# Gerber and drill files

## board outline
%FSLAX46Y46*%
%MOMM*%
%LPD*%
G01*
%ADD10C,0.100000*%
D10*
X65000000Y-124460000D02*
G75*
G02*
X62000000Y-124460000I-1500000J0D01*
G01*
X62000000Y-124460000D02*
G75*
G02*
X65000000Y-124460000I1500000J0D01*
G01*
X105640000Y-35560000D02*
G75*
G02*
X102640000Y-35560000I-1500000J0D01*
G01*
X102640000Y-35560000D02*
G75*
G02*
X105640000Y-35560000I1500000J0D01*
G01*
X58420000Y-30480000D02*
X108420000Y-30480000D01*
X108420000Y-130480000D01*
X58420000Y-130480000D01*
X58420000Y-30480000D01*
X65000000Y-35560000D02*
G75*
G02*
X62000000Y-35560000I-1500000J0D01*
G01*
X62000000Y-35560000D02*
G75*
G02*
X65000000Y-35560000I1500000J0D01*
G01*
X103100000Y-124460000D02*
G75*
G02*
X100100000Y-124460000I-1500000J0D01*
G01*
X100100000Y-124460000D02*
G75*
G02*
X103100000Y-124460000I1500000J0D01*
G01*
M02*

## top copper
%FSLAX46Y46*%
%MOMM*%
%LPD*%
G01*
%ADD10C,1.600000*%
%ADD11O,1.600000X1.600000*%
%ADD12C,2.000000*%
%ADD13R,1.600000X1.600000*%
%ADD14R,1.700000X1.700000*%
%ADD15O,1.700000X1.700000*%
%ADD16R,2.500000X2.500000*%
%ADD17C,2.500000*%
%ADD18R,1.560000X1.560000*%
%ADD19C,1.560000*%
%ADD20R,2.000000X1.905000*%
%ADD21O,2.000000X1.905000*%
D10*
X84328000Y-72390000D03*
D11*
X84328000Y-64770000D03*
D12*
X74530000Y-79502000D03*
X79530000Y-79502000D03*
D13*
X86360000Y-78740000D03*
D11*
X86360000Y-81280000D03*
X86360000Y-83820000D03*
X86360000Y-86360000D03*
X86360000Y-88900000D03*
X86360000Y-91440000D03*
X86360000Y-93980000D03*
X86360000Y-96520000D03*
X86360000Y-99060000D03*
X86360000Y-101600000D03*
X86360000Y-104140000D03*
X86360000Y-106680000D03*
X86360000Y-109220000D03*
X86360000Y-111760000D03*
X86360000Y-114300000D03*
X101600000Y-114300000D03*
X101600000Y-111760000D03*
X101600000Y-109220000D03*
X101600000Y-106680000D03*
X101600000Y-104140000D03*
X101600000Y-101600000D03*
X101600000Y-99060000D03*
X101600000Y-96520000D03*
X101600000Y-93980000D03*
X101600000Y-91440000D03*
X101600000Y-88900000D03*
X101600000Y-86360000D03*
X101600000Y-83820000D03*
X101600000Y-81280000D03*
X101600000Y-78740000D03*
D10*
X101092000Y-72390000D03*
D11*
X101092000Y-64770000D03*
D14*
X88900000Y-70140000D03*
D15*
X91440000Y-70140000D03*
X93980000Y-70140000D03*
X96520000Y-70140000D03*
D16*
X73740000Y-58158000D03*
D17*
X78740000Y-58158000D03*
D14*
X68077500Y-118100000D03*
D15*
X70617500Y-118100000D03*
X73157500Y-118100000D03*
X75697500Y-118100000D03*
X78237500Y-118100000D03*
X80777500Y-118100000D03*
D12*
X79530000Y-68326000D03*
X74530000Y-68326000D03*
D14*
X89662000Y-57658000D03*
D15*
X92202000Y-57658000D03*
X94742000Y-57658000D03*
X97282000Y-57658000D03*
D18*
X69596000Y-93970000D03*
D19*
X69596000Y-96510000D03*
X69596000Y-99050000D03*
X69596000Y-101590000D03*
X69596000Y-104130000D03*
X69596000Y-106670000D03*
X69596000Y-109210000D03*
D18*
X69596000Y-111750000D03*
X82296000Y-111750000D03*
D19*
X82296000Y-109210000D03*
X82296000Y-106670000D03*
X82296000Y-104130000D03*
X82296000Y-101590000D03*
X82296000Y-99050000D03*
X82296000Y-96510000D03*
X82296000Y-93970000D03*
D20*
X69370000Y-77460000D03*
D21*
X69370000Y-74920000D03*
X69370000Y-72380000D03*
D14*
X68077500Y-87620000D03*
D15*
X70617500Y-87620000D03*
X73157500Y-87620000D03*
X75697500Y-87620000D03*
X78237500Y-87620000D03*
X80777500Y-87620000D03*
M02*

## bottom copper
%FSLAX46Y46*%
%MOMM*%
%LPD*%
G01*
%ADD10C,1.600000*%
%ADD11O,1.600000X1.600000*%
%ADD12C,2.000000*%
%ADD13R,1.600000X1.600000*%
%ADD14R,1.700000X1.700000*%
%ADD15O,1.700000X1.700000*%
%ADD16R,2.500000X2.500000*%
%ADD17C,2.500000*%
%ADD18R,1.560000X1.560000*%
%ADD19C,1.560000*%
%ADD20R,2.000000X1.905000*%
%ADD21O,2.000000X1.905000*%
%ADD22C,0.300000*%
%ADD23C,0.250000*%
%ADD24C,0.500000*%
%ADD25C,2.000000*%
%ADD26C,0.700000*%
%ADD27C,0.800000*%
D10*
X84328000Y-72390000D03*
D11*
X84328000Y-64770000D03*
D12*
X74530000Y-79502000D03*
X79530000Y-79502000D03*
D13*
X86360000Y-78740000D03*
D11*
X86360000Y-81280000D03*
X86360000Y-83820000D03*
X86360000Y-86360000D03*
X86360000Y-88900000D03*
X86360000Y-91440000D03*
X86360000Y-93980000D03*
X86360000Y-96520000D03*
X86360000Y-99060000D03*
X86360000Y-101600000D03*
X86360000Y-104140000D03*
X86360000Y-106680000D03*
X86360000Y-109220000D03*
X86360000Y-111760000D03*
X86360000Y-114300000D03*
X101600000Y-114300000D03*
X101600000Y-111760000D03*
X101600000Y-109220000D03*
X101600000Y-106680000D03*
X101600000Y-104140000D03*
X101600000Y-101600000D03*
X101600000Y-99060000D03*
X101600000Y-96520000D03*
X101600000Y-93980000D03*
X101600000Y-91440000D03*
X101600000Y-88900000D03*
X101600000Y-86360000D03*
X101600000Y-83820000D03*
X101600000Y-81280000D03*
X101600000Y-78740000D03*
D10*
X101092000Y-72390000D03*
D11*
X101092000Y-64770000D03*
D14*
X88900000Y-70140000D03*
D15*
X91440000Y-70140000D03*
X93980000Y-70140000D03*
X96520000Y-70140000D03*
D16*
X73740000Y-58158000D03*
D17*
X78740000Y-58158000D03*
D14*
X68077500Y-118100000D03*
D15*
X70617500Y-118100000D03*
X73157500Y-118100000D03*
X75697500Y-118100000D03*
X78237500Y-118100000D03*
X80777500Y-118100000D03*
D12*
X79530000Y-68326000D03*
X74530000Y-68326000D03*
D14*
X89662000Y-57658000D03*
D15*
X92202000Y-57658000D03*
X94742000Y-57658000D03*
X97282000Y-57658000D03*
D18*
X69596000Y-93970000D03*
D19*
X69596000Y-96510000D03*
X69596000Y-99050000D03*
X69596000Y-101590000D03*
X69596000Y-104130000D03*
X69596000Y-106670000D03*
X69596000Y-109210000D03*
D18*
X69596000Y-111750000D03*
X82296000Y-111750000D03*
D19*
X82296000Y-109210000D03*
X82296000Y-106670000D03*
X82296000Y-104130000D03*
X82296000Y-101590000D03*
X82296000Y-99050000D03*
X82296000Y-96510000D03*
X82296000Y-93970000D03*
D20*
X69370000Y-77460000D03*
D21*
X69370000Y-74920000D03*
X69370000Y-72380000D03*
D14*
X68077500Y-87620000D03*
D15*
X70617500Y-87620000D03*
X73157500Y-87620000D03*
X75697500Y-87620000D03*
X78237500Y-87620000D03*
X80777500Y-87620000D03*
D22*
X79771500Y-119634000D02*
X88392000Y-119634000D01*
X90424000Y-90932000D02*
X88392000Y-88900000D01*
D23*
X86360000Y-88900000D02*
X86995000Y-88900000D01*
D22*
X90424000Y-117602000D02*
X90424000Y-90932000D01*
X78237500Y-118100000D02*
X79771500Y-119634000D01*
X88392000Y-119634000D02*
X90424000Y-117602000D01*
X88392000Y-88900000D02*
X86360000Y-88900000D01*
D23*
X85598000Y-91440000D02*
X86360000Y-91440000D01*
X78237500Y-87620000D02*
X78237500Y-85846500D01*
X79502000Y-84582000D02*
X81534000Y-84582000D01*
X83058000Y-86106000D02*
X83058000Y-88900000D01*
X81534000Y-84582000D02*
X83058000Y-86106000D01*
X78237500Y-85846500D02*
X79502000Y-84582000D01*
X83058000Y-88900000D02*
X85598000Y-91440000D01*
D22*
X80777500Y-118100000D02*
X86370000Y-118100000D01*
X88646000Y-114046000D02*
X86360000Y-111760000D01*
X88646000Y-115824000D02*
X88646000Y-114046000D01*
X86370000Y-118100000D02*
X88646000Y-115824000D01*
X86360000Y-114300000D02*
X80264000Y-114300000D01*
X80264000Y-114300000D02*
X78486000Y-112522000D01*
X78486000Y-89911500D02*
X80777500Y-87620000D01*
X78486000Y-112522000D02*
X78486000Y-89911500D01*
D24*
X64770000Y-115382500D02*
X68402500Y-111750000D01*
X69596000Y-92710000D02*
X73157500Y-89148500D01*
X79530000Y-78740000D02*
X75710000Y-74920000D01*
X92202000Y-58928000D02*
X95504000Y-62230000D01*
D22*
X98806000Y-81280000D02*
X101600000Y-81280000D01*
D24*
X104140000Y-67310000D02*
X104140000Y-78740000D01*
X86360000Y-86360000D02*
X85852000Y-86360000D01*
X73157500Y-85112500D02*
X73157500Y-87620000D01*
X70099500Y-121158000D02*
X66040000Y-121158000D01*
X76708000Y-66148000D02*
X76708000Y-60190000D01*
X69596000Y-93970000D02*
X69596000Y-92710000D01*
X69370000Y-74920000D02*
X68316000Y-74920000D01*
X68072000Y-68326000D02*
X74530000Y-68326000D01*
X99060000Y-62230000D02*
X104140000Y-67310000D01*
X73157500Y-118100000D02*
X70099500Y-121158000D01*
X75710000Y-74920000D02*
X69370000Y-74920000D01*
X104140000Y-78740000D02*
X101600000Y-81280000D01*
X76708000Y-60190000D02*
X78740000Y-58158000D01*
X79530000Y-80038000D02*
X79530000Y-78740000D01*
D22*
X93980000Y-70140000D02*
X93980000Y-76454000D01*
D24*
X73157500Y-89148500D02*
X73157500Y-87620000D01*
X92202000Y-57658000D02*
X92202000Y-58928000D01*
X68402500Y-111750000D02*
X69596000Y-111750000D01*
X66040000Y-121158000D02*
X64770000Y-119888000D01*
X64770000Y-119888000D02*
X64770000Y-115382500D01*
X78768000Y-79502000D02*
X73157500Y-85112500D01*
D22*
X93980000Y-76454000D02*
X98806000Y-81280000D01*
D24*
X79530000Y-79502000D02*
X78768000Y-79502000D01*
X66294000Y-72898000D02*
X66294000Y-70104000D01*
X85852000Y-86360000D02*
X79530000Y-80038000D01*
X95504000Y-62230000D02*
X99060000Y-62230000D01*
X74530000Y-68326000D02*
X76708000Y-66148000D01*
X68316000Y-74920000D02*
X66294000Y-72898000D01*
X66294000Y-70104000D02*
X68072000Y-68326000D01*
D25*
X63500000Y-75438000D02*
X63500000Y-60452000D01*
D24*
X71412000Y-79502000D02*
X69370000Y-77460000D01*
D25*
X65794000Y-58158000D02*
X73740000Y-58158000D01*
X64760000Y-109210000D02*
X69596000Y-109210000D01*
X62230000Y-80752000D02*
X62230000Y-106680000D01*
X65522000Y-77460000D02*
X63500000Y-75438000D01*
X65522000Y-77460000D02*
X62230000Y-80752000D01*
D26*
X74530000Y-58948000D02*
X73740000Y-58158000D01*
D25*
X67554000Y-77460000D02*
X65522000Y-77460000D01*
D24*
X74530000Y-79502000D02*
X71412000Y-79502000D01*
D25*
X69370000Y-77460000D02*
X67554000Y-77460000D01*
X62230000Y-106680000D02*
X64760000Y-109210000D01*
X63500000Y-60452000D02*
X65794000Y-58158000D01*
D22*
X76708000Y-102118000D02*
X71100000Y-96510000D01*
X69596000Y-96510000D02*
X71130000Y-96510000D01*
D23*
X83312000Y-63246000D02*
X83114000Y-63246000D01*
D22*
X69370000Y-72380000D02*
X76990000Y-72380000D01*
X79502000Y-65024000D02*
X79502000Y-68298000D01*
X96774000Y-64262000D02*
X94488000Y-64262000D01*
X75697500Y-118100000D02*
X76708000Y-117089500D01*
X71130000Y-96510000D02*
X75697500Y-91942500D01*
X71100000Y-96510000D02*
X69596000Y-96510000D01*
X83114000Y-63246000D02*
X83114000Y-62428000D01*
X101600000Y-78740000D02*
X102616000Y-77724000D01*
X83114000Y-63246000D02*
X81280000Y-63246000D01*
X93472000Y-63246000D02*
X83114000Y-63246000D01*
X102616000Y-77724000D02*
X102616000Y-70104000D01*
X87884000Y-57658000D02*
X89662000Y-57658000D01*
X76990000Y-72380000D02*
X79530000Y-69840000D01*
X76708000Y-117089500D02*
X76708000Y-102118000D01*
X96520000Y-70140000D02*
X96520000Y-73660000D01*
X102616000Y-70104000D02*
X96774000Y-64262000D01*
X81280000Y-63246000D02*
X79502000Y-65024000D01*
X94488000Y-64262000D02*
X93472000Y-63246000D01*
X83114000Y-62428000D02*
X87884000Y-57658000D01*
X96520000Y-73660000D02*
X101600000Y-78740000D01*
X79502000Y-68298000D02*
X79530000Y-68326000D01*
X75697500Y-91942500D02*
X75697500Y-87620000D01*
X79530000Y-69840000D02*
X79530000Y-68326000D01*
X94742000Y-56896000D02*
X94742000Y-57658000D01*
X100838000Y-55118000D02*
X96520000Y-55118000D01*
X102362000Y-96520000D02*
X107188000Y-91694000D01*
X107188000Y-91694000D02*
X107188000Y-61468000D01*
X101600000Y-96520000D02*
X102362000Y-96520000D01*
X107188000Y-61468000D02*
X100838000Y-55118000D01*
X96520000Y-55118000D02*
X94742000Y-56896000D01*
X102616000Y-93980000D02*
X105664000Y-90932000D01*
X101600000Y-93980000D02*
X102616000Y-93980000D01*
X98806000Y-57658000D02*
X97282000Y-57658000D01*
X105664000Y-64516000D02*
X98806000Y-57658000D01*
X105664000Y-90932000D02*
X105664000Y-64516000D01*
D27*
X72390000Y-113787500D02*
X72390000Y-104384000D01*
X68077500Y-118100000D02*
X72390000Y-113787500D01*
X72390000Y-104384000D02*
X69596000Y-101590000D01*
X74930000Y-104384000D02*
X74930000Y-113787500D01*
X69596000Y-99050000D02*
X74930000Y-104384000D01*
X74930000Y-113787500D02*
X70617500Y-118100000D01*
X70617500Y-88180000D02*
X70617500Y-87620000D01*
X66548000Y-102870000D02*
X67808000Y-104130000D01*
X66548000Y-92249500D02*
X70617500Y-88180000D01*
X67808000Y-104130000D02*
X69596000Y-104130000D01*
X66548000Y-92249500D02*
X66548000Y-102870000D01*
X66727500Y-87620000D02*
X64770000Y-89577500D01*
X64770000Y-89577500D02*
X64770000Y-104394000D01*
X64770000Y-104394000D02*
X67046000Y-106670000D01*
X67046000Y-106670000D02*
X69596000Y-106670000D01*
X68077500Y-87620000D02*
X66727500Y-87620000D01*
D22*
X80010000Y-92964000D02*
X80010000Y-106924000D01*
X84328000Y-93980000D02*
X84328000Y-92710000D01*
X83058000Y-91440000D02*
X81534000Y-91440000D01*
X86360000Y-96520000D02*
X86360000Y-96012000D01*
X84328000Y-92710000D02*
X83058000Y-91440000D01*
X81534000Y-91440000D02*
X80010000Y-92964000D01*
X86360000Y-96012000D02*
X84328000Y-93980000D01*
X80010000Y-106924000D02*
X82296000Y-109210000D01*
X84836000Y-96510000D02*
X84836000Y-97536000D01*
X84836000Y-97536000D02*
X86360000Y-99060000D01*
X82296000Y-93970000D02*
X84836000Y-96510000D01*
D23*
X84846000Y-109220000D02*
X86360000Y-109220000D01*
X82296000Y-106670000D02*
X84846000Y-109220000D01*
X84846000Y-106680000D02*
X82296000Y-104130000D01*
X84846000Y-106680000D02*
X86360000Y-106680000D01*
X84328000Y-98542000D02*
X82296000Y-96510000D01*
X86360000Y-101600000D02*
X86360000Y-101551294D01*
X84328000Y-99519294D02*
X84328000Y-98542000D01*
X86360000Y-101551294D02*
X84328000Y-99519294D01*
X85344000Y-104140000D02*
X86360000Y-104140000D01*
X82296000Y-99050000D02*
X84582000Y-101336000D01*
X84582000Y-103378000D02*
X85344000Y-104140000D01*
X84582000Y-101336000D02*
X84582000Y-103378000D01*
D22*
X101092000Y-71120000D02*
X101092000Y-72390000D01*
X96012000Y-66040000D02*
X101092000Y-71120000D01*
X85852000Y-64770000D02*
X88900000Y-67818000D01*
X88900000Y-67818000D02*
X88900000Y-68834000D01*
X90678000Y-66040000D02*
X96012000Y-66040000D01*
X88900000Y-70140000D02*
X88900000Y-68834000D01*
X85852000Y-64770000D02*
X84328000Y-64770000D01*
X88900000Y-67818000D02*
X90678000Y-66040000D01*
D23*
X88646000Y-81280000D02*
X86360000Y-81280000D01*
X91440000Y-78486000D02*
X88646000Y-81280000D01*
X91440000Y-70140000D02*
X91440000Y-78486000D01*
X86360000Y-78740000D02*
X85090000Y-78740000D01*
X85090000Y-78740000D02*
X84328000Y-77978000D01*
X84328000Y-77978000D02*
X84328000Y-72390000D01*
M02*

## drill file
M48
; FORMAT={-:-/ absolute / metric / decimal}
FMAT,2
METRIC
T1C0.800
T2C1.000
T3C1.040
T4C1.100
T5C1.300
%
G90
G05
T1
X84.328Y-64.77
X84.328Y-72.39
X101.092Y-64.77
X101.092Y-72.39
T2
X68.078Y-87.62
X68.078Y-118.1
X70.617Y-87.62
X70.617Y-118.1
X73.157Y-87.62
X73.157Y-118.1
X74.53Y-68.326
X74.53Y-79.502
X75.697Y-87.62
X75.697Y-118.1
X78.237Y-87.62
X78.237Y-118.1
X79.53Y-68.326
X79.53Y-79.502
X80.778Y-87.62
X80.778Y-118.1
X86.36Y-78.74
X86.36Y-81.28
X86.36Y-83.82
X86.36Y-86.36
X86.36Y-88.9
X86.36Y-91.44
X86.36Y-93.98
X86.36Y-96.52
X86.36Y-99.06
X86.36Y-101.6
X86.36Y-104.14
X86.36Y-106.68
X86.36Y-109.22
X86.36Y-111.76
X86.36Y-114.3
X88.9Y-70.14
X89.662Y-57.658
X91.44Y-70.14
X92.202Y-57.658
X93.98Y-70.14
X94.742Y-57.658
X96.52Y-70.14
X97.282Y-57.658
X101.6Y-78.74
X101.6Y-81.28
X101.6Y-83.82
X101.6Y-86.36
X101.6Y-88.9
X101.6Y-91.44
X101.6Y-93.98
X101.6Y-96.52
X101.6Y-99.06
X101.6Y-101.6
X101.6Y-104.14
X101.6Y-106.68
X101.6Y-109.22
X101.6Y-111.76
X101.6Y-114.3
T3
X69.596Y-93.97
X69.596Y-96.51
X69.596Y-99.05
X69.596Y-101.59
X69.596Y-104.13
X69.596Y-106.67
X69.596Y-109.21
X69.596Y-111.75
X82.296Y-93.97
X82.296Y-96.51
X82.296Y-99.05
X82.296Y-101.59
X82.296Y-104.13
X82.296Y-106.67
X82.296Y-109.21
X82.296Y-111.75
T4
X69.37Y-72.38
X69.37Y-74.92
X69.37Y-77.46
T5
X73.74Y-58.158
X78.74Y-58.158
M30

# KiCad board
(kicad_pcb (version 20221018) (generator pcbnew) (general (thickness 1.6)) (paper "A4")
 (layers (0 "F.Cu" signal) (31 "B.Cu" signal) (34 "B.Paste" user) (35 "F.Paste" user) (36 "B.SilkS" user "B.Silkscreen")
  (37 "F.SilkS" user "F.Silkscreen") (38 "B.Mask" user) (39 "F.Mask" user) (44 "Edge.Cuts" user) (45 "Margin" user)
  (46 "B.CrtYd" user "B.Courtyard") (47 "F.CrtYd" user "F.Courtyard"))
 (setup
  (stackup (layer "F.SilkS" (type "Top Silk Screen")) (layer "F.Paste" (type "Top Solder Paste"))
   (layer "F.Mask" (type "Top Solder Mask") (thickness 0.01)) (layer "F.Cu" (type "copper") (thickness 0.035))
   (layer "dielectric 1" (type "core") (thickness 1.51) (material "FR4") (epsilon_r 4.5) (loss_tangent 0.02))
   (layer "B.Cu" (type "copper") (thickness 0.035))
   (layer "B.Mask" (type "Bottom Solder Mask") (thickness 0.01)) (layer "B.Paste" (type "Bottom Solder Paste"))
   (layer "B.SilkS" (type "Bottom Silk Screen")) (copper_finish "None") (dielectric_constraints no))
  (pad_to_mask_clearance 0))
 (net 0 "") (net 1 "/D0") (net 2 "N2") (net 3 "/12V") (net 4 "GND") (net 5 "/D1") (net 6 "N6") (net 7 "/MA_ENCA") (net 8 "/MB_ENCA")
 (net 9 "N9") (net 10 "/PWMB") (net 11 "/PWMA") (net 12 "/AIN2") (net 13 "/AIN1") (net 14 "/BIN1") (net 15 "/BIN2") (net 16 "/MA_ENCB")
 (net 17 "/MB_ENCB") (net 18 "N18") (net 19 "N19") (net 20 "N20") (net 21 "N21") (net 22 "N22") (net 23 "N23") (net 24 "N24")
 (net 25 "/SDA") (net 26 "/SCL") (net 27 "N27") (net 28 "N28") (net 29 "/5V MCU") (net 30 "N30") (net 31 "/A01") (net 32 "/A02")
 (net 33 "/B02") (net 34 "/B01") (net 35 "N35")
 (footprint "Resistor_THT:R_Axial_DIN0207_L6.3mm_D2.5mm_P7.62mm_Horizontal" (layer "F.Cu") (at 84.328 72.39 90)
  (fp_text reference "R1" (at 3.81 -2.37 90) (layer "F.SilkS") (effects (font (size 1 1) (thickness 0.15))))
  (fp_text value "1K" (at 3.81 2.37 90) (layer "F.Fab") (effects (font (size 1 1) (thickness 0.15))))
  (pad "1" thru_hole circle (at 0 0 90) (size 1.6 1.6) (drill 0.8) (layers "*.Cu" "*.Mask") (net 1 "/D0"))
  (pad "2" thru_hole oval (at 7.62 0 90) (size 1.6 1.6) (drill 0.8) (layers "*.Cu" "*.Mask") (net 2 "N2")))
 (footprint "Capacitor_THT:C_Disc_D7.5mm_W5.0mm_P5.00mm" (layer "F.Cu") (at 74.53 79.502)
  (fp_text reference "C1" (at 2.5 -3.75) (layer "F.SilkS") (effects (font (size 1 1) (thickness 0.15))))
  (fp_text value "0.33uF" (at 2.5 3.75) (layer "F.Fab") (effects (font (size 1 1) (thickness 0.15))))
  (pad "1" thru_hole circle (at 0 0) (size 2 2) (drill 1) (layers "*.Cu" "*.Mask") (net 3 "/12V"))
  (pad "2" thru_hole circle (at 5 0) (size 2 2) (drill 1) (layers "*.Cu" "*.Mask") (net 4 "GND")))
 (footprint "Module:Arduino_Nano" (layer "F.Cu") (at 86.36 78.74)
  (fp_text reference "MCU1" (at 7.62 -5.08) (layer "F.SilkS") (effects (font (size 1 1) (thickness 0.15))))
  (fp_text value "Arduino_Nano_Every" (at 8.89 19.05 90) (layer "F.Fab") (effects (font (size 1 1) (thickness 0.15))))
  (pad "1" thru_hole rect (at 0 0) (size 1.6 1.6) (drill 1) (layers "*.Cu" "*.Mask") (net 1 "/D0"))
  (pad "2" thru_hole oval (at 0 2.54) (size 1.6 1.6) (drill 1) (layers "*.Cu" "*.Mask") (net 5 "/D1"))
  (pad "3" thru_hole oval (at 0 5.08) (size 1.6 1.6) (drill 1) (layers "*.Cu" "*.Mask") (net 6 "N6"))
  (pad "4" thru_hole oval (at 0 7.62) (size 1.6 1.6) (drill 1) (layers "*.Cu" "*.Mask") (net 4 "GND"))
  (pad "5" thru_hole oval (at 0 10.16) (size 1.6 1.6) (drill 1) (layers "*.Cu" "*.Mask") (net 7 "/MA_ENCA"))
  (pad "6" thru_hole oval (at 0 12.7) (size 1.6 1.6) (drill 1) (layers "*.Cu" "*.Mask") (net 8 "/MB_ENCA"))
  (pad "7" thru_hole oval (at 0 15.24) (size 1.6 1.6) (drill 1) (layers "*.Cu" "*.Mask") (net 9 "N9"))
  (pad "8" thru_hole oval (at 0 17.78) (size 1.6 1.6) (drill 1) (layers "*.Cu" "*.Mask") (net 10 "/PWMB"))
  (pad "9" thru_hole oval (at 0 20.32) (size 1.6 1.6) (drill 1) (layers "*.Cu" "*.Mask") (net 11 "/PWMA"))
  (pad "10" thru_hole oval (at 0 22.86) (size 1.6 1.6) (drill 1) (layers "*.Cu" "*.Mask") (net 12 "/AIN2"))
  (pad "11" thru_hole oval (at 0 25.4) (size 1.6 1.6) (drill 1) (layers "*.Cu" "*.Mask") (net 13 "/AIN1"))
  (pad "12" thru_hole oval (at 0 27.94) (size 1.6 1.6) (drill 1) (layers "*.Cu" "*.Mask") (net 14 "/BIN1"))
  (pad "13" thru_hole oval (at 0 30.48) (size 1.6 1.6) (drill 1) (layers "*.Cu" "*.Mask") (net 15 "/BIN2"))
  (pad "14" thru_hole oval (at 0 33.02) (size 1.6 1.6) (drill 1) (layers "*.Cu" "*.Mask") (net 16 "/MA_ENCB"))
  (pad "15" thru_hole oval (at 0 35.56) (size 1.6 1.6) (drill 1) (layers "*.Cu" "*.Mask") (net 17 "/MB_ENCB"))
  (pad "16" thru_hole oval (at 15.24 35.56) (size 1.6 1.6) (drill 1) (layers "*.Cu" "*.Mask") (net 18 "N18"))
  (pad "17" thru_hole oval (at 15.24 33.02) (size 1.6 1.6) (drill 1) (layers "*.Cu" "*.Mask") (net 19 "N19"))
  (pad "18" thru_hole oval (at 15.24 30.48) (size 1.6 1.6) (drill 1) (layers "*.Cu" "*.Mask") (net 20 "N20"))
  (pad "19" thru_hole oval (at 15.24 27.94) (size 1.6 1.6) (drill 1) (layers "*.Cu" "*.Mask") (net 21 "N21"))
  (pad "20" thru_hole oval (at 15.24 25.4) (size 1.6 1.6) (drill 1) (layers "*.Cu" "*.Mask") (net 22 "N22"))
  (pad "21" thru_hole oval (at 15.24 22.86) (size 1.6 1.6) (drill 1) (layers "*.Cu" "*.Mask") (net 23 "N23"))
  (pad "22" thru_hole oval (at 15.24 20.32) (size 1.6 1.6) (drill 1) (layers "*.Cu" "*.Mask") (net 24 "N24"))
  (pad "23" thru_hole oval (at 15.24 17.78) (size 1.6 1.6) (drill 1) (layers "*.Cu" "*.Mask") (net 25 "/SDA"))
  (pad "24" thru_hole oval (at 15.24 15.24) (size 1.6 1.6) (drill 1) (layers "*.Cu" "*.Mask") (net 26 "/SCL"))
  (pad "25" thru_hole oval (at 15.24 12.7) (size 1.6 1.6) (drill 1) (layers "*.Cu" "*.Mask") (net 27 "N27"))
  (pad "26" thru_hole oval (at 15.24 10.16) (size 1.6 1.6) (drill 1) (layers "*.Cu" "*.Mask") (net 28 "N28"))
  (pad "27" thru_hole oval (at 15.24 7.62) (size 1.6 1.6) (drill 1) (layers "*.Cu" "*.Mask") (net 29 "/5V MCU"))
  (pad "28" thru_hole oval (at 15.24 5.08) (size 1.6 1.6) (drill 1) (layers "*.Cu" "*.Mask") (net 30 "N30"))
  (pad "29" thru_hole oval (at 15.24 2.54) (size 1.6 1.6) (drill 1) (layers "*.Cu" "*.Mask") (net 4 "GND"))
  (pad "30" thru_hole oval (at 15.24 0) (size 1.6 1.6) (drill 1) (layers "*.Cu" "*.Mask") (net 29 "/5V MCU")))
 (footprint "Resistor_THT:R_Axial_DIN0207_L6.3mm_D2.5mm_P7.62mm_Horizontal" (layer "F.Cu") (at 101.092 72.39 90)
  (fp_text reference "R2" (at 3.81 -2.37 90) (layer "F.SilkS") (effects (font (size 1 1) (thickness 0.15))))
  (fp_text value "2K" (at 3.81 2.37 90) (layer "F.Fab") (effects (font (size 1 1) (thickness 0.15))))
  (pad "1" thru_hole circle (at 0 0 90) (size 1.6 1.6) (drill 0.8) (layers "*.Cu" "*.Mask") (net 2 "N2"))
  (pad "2" thru_hole oval (at 7.62 0 90) (size 1.6 1.6) (drill 0.8) (layers "*.Cu" "*.Mask") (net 4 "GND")))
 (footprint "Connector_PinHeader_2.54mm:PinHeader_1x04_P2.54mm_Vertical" (layer "F.Cu") (at 88.9 70.14 90)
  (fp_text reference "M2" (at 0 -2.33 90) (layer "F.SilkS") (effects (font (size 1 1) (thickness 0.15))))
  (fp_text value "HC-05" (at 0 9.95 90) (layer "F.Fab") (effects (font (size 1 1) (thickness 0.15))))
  (pad "1" thru_hole rect (at 0 0 90) (size 1.7 1.7) (drill 1) (layers "*.Cu" "*.Mask") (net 2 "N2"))
  (pad "2" thru_hole oval (at 0 2.54 90) (size 1.7 1.7) (drill 1) (layers "*.Cu" "*.Mask") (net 5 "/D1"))
  (pad "3" thru_hole oval (at 0 5.08 90) (size 1.7 1.7) (drill 1) (layers "*.Cu" "*.Mask") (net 4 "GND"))
  (pad "4" thru_hole oval (at 0 7.62 90) (size 1.7 1.7) (drill 1) (layers "*.Cu" "*.Mask") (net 29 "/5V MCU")))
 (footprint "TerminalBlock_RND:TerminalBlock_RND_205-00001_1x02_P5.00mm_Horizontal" (layer "F.Cu") (at 73.74 58.158)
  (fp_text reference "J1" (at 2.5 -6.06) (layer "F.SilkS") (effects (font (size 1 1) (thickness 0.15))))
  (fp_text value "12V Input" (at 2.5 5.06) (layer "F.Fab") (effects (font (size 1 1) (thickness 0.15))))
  (pad "1" thru_hole rect (at 0 0) (size 2.5 2.5) (drill 1.3) (layers "*.Cu" "*.Mask") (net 3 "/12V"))
  (pad "2" thru_hole circle (at 5 0) (size 2.5 2.5) (drill 1.3) (layers "*.Cu" "*.Mask") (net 4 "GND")))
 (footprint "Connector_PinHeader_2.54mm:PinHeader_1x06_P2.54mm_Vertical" (layer "F.Cu") (at 68.0775 118.1 90)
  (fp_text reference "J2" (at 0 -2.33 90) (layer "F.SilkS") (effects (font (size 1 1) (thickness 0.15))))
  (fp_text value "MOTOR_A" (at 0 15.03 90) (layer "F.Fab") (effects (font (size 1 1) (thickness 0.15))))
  (pad "1" thru_hole rect (at 0 0 90) (size 1.7 1.7) (drill 1) (layers "*.Cu" "*.Mask") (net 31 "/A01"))
  (pad "2" thru_hole oval (at 0 2.54 90) (size 1.7 1.7) (drill 1) (layers "*.Cu" "*.Mask") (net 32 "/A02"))
  (pad "3" thru_hole oval (at 0 5.08 90) (size 1.7 1.7) (drill 1) (layers "*.Cu" "*.Mask") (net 4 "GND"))
  (pad "4" thru_hole oval (at 0 7.62 90) (size 1.7 1.7) (drill 1) (layers "*.Cu" "*.Mask") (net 29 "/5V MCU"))
  (pad "5" thru_hole oval (at 0 10.16 90) (size 1.7 1.7) (drill 1) (layers "*.Cu" "*.Mask") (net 7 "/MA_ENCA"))
  (pad "6" thru_hole oval (at 0 12.7 90) (size 1.7 1.7) (drill 1) (layers "*.Cu" "*.Mask") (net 16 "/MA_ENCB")))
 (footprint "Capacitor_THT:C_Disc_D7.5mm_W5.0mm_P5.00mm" (layer "F.Cu") (at 79.53 68.326 180)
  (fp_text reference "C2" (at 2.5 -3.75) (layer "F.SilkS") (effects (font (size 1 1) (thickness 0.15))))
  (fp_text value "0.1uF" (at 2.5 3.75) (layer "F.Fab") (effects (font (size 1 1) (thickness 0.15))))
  (pad "1" thru_hole circle (at 0 0 180) (size 2 2) (drill 1) (layers "*.Cu" "*.Mask") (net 29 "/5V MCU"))
  (pad "2" thru_hole circle (at 5 0 180) (size 2 2) (drill 1) (layers "*.Cu" "*.Mask") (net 4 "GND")))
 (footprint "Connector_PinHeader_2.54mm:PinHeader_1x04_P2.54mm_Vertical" (layer "F.Cu") (at 89.662 57.658 90)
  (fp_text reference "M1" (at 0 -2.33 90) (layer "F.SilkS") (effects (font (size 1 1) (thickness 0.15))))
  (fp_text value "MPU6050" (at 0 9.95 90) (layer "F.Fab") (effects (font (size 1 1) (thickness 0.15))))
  (pad "1" thru_hole rect (at 0 0 90) (size 1.7 1.7) (drill 1) (layers "*.Cu" "*.Mask") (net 29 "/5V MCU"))
  (pad "2" thru_hole oval (at 0 2.54 90) (size 1.7 1.7) (drill 1) (layers "*.Cu" "*.Mask") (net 4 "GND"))
  (pad "3" thru_hole oval (at 0 5.08 90) (size 1.7 1.7) (drill 1) (layers "*.Cu" "*.Mask") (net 25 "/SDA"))
  (pad "4" thru_hole oval (at 0 7.62 90) (size 1.7 1.7) (drill 1) (layers "*.Cu" "*.Mask") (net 26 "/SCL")))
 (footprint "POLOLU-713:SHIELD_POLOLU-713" (layer "F.Cu") (at 75.946 102.86)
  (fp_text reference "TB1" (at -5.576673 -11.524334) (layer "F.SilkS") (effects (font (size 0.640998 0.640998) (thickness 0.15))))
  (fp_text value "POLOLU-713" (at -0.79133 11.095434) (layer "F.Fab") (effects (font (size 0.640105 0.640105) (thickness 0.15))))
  (pad "1" thru_hole rect (at -6.35 -8.89) (size 1.56 1.56) (drill 1.04) (layers "*.Cu" "*.Mask") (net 4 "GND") (solder_mask_margin 0.102))
  (pad "2" thru_hole circle (at -6.35 -6.35) (size 1.56 1.56) (drill 1.04) (layers "*.Cu" "*.Mask") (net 29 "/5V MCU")
   (solder_mask_margin 0.102))
  (pad "3" thru_hole circle (at -6.35 -3.81) (size 1.56 1.56) (drill 1.04) (layers "*.Cu" "*.Mask") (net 32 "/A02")
   (solder_mask_margin 0.102))
  (pad "4" thru_hole circle (at -6.35 -1.27) (size 1.56 1.56) (drill 1.04) (layers "*.Cu" "*.Mask") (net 31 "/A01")
   (solder_mask_margin 0.102))
  (pad "5" thru_hole circle (at -6.35 1.27) (size 1.56 1.56) (drill 1.04) (layers "*.Cu" "*.Mask") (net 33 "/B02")
   (solder_mask_margin 0.102))
  (pad "6" thru_hole circle (at -6.35 3.81) (size 1.56 1.56) (drill 1.04) (layers "*.Cu" "*.Mask") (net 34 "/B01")
   (solder_mask_margin 0.102))
  (pad "7" thru_hole circle (at -6.35 6.35) (size 1.56 1.56) (drill 1.04) (layers "*.Cu" "*.Mask") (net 3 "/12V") (solder_mask_margin 0.102))
  (pad "8" thru_hole rect (at -6.35 8.89) (size 1.56 1.56) (drill 1.04) (layers "*.Cu" "*.Mask") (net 4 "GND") (solder_mask_margin 0.102))
  (pad "9" thru_hole rect (at 6.35 8.89) (size 1.56 1.56) (drill 1.04) (layers "*.Cu" "*.Mask") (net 4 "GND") (solder_mask_margin 0.102))
  (pad "10" thru_hole circle (at 6.35 6.35) (size 1.56 1.56) (drill 1.04) (layers "*.Cu" "*.Mask") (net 10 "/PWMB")
   (solder_mask_margin 0.102))
  (pad "11" thru_hole circle (at 6.35 3.81) (size 1.56 1.56) (drill 1.04) (layers "*.Cu" "*.Mask") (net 15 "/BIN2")
   (solder_mask_margin 0.102))
  (pad "12" thru_hole circle (at 6.35 1.27) (size 1.56 1.56) (drill 1.04) (layers "*.Cu" "*.Mask") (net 14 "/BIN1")
   (solder_mask_margin 0.102))
  (pad "13" thru_hole circle (at 6.35 -1.27) (size 1.56 1.56) (drill 1.04) (layers "*.Cu" "*.Mask") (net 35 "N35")
   (solder_mask_margin 0.102))
  (pad "14" thru_hole circle (at 6.35 -3.81) (size 1.56 1.56) (drill 1.04) (layers "*.Cu" "*.Mask") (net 13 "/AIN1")
   (solder_mask_margin 0.102))
  (pad "15" thru_hole circle (at 6.35 -6.35) (size 1.56 1.56) (drill 1.04) (layers "*.Cu" "*.Mask") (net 12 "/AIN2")
   (solder_mask_margin 0.102))
  (pad "16" thru_hole circle (at 6.35 -8.89) (size 1.56 1.56) (drill 1.04) (layers "*.Cu" "*.Mask") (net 11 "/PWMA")
   (solder_mask_margin 0.102)))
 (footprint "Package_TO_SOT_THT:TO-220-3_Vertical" (layer "F.Cu") (at 69.37 77.46 90)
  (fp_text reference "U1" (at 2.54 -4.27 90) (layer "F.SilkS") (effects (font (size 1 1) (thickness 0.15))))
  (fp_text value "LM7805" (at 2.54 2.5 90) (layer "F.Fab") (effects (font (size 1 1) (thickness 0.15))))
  (pad "1" thru_hole rect (at 0 0 90) (size 1.905 2) (drill 1.1) (layers "*.Cu" "*.Mask") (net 3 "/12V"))
  (pad "2" thru_hole oval (at 2.54 0 90) (size 1.905 2) (drill 1.1) (layers "*.Cu" "*.Mask") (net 4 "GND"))
  (pad "3" thru_hole oval (at 5.08 0 90) (size 1.905 2) (drill 1.1) (layers "*.Cu" "*.Mask") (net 29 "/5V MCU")))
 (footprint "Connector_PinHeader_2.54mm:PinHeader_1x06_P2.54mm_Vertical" (layer "F.Cu") (at 68.0775 87.62 90)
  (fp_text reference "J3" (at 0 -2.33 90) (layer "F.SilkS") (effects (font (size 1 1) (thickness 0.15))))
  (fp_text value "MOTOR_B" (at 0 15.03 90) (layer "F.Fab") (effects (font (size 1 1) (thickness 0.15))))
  (pad "1" thru_hole rect (at 0 0 90) (size 1.7 1.7) (drill 1) (layers "*.Cu" "*.Mask") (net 34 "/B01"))
  (pad "2" thru_hole oval (at 0 2.54 90) (size 1.7 1.7) (drill 1) (layers "*.Cu" "*.Mask") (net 33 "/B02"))
  (pad "3" thru_hole oval (at 0 5.08 90) (size 1.7 1.7) (drill 1) (layers "*.Cu" "*.Mask") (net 4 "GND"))
  (pad "4" thru_hole oval (at 0 7.62 90) (size 1.7 1.7) (drill 1) (layers "*.Cu" "*.Mask") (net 29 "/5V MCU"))
  (pad "5" thru_hole oval (at 0 10.16 90) (size 1.7 1.7) (drill 1) (layers "*.Cu" "*.Mask") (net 8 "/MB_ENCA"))
  (pad "6" thru_hole oval (at 0 12.7 90) (size 1.7 1.7) (drill 1) (layers "*.Cu" "*.Mask") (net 17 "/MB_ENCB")))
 (gr_circle (center 63.5 124.46) (end 65 124.46) (stroke (width 0.1) (type default)) (fill none) (layer "Edge.Cuts"))
 (gr_circle (center 104.14 35.56) (end 105.64 35.56) (stroke (width 0.1) (type default)) (fill none) (layer "Edge.Cuts"))
 (gr_rect (start 58.42 30.48) (end 108.42 130.48) (stroke (width 0.1) (type default)) (fill none) (layer "Edge.Cuts"))
 (gr_circle (center 63.5 35.56) (end 65 35.56) (stroke (width 0.1) (type default)) (fill none) (layer "Edge.Cuts"))
 (gr_circle (center 101.6 124.46) (end 103.1 124.46) (stroke (width 0.1) (type default)) (fill none) (layer "Edge.Cuts"))
 (segment (start 79.7715 119.634) (end 88.392 119.634) (width 0.3) (layer "B.Cu") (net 7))
 (segment (start 90.424 90.932) (end 88.392 88.9) (width 0.3) (layer "B.Cu") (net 7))
 (segment (start 86.36 88.9) (end 86.995 88.9) (width 0.25) (layer "B.Cu") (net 7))
 (segment (start 90.424 117.602) (end 90.424 90.932) (width 0.3) (layer "B.Cu") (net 7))
 (segment (start 78.2375 118.1) (end 79.7715 119.634) (width 0.3) (layer "B.Cu") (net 7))
 (segment (start 88.392 119.634) (end 90.424 117.602) (width 0.3) (layer "B.Cu") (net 7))
 (segment (start 88.392 88.9) (end 86.36 88.9) (width 0.3) (layer "B.Cu") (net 7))
 (segment (start 85.598 91.44) (end 86.36 91.44) (width 0.25) (layer "B.Cu") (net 8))
 (segment (start 78.2375 87.62) (end 78.2375 85.8465) (width 0.25) (layer "B.Cu") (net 8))
 (segment (start 79.502 84.582) (end 81.534 84.582) (width 0.25) (layer "B.Cu") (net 8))
 (segment (start 83.058 86.106) (end 83.058 88.9) (width 0.25) (layer "B.Cu") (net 8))
 (segment (start 81.534 84.582) (end 83.058 86.106) (width 0.25) (layer "B.Cu") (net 8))
 (segment (start 78.2375 85.8465) (end 79.502 84.582) (width 0.25) (layer "B.Cu") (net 8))
 (segment (start 83.058 88.9) (end 85.598 91.44) (width 0.25) (layer "B.Cu") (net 8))
 (segment (start 80.7775 118.1) (end 86.37 118.1) (width 0.3) (layer "B.Cu") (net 16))
 (segment (start 88.646 114.046) (end 86.36 111.76) (width 0.3) (layer "B.Cu") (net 16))
 (segment (start 88.646 115.824) (end 88.646 114.046) (width 0.3) (layer "B.Cu") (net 16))
 (segment (start 86.37 118.1) (end 88.646 115.824) (width 0.3) (layer "B.Cu") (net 16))
 (segment (start 86.36 114.3) (end 80.264 114.3) (width 0.3) (layer "B.Cu") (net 17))
 (segment (start 80.264 114.3) (end 78.486 112.522) (width 0.3) (layer "B.Cu") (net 17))
 (segment (start 78.486 89.9115) (end 80.7775 87.62) (width 0.3) (layer "B.Cu") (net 17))
 (segment (start 78.486 112.522) (end 78.486 89.9115) (width 0.3) (layer "B.Cu") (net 17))
 (segment (start 64.77 115.3825) (end 68.4025 111.75) (width 0.5) (layer "B.Cu") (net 4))
 (segment (start 69.596 92.71) (end 73.1575 89.1485) (width 0.5) (layer "B.Cu") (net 4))
 (segment (start 79.53 78.74) (end 75.71 74.92) (width 0.5) (layer "B.Cu") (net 4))
 (segment (start 92.202 58.928) (end 95.504 62.23) (width 0.5) (layer "B.Cu") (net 4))
 (segment (start 98.806 81.28) (end 101.6 81.28) (width 0.3) (layer "B.Cu") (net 4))
 (segment (start 104.14 67.31) (end 104.14 78.74) (width 0.5) (layer "B.Cu") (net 4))
 (segment (start 86.36 86.36) (end 85.852 86.36) (width 0.5) (layer "B.Cu") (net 4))
 (segment (start 73.1575 85.1125) (end 73.1575 87.62) (width 0.5) (layer "B.Cu") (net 4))
 (segment (start 70.0995 121.158) (end 66.04 121.158) (width 0.5) (layer "B.Cu") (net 4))
 (segment (start 76.708 66.148) (end 76.708 60.19) (width 0.5) (layer "B.Cu") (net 4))
 (segment (start 69.596 93.97) (end 69.596 92.71) (width 0.5) (layer "B.Cu") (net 4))
 (segment (start 69.37 74.92) (end 68.316 74.92) (width 0.5) (layer "B.Cu") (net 4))
 (segment (start 68.072 68.326) (end 74.53 68.326) (width 0.5) (layer "B.Cu") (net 4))
 (segment (start 99.06 62.23) (end 104.14 67.31) (width 0.5) (layer "B.Cu") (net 4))
 (segment (start 73.1575 118.1) (end 70.0995 121.158) (width 0.5) (layer "B.Cu") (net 4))
 (segment (start 75.71 74.92) (end 69.37 74.92) (width 0.5) (layer "B.Cu") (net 4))
 (segment (start 104.14 78.74) (end 101.6 81.28) (width 0.5) (layer "B.Cu") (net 4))
 (segment (start 76.708 60.19) (end 78.74 58.158) (width 0.5) (layer "B.Cu") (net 4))
 (segment (start 79.53 80.038) (end 79.53 78.74) (width 0.5) (layer "B.Cu") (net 4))
 (segment (start 93.98 70.14) (end 93.98 76.454) (width 0.3) (layer "B.Cu") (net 4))
 (segment (start 73.1575 89.1485) (end 73.1575 87.62) (width 0.5) (layer "B.Cu") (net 4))
 (segment (start 92.202 57.658) (end 92.202 58.928) (width 0.5) (layer "B.Cu") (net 4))
 (segment (start 68.4025 111.75) (end 69.596 111.75) (width 0.5) (layer "B.Cu") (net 4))
 (segment (start 66.04 121.158) (end 64.77 119.888) (width 0.5) (layer "B.Cu") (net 4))
 (segment (start 64.77 119.888) (end 64.77 115.3825) (width 0.5) (layer "B.Cu") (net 4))
 (segment (start 78.768 79.502) (end 73.1575 85.1125) (width 0.5) (layer "B.Cu") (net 4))
 (segment (start 93.98 76.454) (end 98.806 81.28) (width 0.3) (layer "B.Cu") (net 4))
 (segment (start 79.53 79.502) (end 78.768 79.502) (width 0.5) (layer "B.Cu") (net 4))
 (segment (start 66.294 72.898) (end 66.294 70.104) (width 0.5) (layer "B.Cu") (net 4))
 (segment (start 85.852 86.36) (end 79.53 80.038) (width 0.5) (layer "B.Cu") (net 4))
 (segment (start 95.504 62.23) (end 99.06 62.23) (width 0.5) (layer "B.Cu") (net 4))
 (segment (start 74.53 68.326) (end 76.708 66.148) (width 0.5) (layer "B.Cu") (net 4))
 (segment (start 68.316 74.92) (end 66.294 72.898) (width 0.5) (layer "B.Cu") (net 4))
 (segment (start 66.294 70.104) (end 68.072 68.326) (width 0.5) (layer "B.Cu") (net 4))
 (segment (start 63.5 75.438) (end 63.5 60.452) (width 2) (layer "B.Cu") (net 3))
 (segment (start 71.412 79.502) (end 69.37 77.46) (width 0.5) (layer "B.Cu") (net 3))
 (segment (start 65.794 58.158) (end 73.74 58.158) (width 2) (layer "B.Cu") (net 3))
 (segment (start 64.76 109.21) (end 69.596 109.21) (width 2) (layer "B.Cu") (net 3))
 (segment (start 62.23 80.752) (end 62.23 106.68) (width 2) (layer "B.Cu") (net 3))
 (segment (start 65.522 77.46) (end 63.5 75.438) (width 2) (layer "B.Cu") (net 3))
 (segment (start 65.522 77.46) (end 62.23 80.752) (width 2) (layer "B.Cu") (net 3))
 (segment (start 74.53 58.948) (end 73.74 58.158) (width 0.7) (layer "B.Cu") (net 3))
 (segment (start 67.554 77.46) (end 65.522 77.46) (width 2) (layer "B.Cu") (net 3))
 (segment (start 74.53 79.502) (end 71.412 79.502) (width 0.5) (layer "B.Cu") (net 3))
 (segment (start 69.37 77.46) (end 67.554 77.46) (width 2) (layer "B.Cu") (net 3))
 (segment (start 62.23 106.68) (end 64.76 109.21) (width 2) (layer "B.Cu") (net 3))
 (segment (start 63.5 60.452) (end 65.794 58.158) (width 2) (layer "B.Cu") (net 3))
 (segment (start 76.708 102.118) (end 71.1 96.51) (width 0.3) (layer "B.Cu") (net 29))
 (segment (start 69.596 96.51) (end 71.13 96.51) (width 0.3) (layer "B.Cu") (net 29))
 (segment (start 83.312 63.246) (end 83.114 63.246) (width 0.25) (layer "B.Cu") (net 29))
 (segment (start 69.37 72.38) (end 76.99 72.38) (width 0.3) (layer "B.Cu") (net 29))
 (segment (start 79.502 65.024) (end 79.502 68.298) (width 0.3) (layer "B.Cu") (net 29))
 (segment (start 96.774 64.262) (end 94.488 64.262) (width 0.3) (layer "B.Cu") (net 29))
 (segment (start 75.6975 118.1) (end 76.708 117.0895) (width 0.3) (layer "B.Cu") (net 29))
 (segment (start 71.13 96.51) (end 75.6975 91.9425) (width 0.3) (layer "B.Cu") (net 29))
 (segment (start 71.1 96.51) (end 69.596 96.51) (width 0.3) (layer "B.Cu") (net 29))
 (segment (start 83.114 63.246) (end 83.114 62.428) (width 0.3) (layer "B.Cu") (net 29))
 (segment (start 101.6 78.74) (end 102.616 77.724) (width 0.3) (layer "B.Cu") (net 29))
 (segment (start 83.114 63.246) (end 81.28 63.246) (width 0.3) (layer "B.Cu") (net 29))
 (segment (start 93.472 63.246) (end 83.114 63.246) (width 0.3) (layer "B.Cu") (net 29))
 (segment (start 102.616 77.724) (end 102.616 70.104) (width 0.3) (layer "B.Cu") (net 29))
 (segment (start 87.884 57.658) (end 89.662 57.658) (width 0.3) (layer "B.Cu") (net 29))
 (segment (start 76.99 72.38) (end 79.53 69.84) (width 0.3) (layer "B.Cu") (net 29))
 (segment (start 76.708 117.0895) (end 76.708 102.118) (width 0.3) (layer "B.Cu") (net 29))
 (segment (start 96.52 70.14) (end 96.52 73.66) (width 0.3) (layer "B.Cu") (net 29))
 (segment (start 102.616 70.104) (end 96.774 64.262) (width 0.3) (layer "B.Cu") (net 29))
 (segment (start 81.28 63.246) (end 79.502 65.024) (width 0.3) (layer "B.Cu") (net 29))
 (segment (start 94.488 64.262) (end 93.472 63.246) (width 0.3) (layer "B.Cu") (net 29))
 (segment (start 83.114 62.428) (end 87.884 57.658) (width 0.3) (layer "B.Cu") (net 29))
 (segment (start 96.52 73.66) (end 101.6 78.74) (width 0.3) (layer "B.Cu") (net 29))
 (segment (start 79.502 68.298) (end 79.53 68.326) (width 0.3) (layer "B.Cu") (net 29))
 (segment (start 75.6975 91.9425) (end 75.6975 87.62) (width 0.3) (layer "B.Cu") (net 29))
 (segment (start 79.53 69.84) (end 79.53 68.326) (width 0.3) (layer "B.Cu") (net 29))
 (segment (start 94.742 56.896) (end 94.742 57.658) (width 0.3) (layer "B.Cu") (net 25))
 (segment (start 100.838 55.118) (end 96.52 55.118) (width 0.3) (layer "B.Cu") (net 25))
 (segment (start 102.362 96.52) (end 107.188 91.694) (width 0.3) (layer "B.Cu") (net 25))
 (segment (start 107.188 91.694) (end 107.188 61.468) (width 0.3) (layer "B.Cu") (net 25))
 (segment (start 101.6 96.52) (end 102.362 96.52) (width 0.3) (layer "B.Cu") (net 25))
 (segment (start 107.188 61.468) (end 100.838 55.118) (width 0.3) (layer "B.Cu") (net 25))
 (segment (start 96.52 55.118) (end 94.742 56.896) (width 0.3) (layer "B.Cu") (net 25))
 (segment (start 102.616 93.98) (end 105.664 90.932) (width 0.3) (layer "B.Cu") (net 26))
 (segment (start 101.6 93.98) (end 102.616 93.98) (width 0.3) (layer "B.Cu") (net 26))
 (segment (start 98.806 57.658) (end 97.282 57.658) (width 0.3) (layer "B.Cu") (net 26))
 (segment (start 105.664 64.516) (end 98.806 57.658) (width 0.3) (layer "B.Cu") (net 26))
 (segment (start 105.664 90.932) (end 105.664 64.516) (width 0.3) (layer "B.Cu") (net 26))
 (segment (start 72.39 113.7875) (end 72.39 104.384) (width 0.8) (layer "B.Cu") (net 31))
 (segment (start 68.0775 118.1) (end 72.39 113.7875) (width 0.8) (layer "B.Cu") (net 31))
 (segment (start 72.39 104.384) (end 69.596 101.59) (width 0.8) (layer "B.Cu") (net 31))
 (segment (start 74.93 104.384) (end 74.93 113.7875) (width 0.8) (layer "B.Cu") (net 32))
 (segment (start 69.596 99.05) (end 74.93 104.384) (width 0.8) (layer "B.Cu") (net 32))
 (segment (start 74.93 113.7875) (end 70.6175 118.1) (width 0.8) (layer "B.Cu") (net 32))
 (segment (start 70.6175 88.18) (end 70.6175 87.62) (width 0.8) (layer "B.Cu") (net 33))
 (segment (start 66.548 102.87) (end 67.808 104.13) (width 0.8) (layer "B.Cu") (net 33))
 (segment (start 66.548 92.2495) (end 70.6175 88.18) (width 0.8) (layer "B.Cu") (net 33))
 (segment (start 67.808 104.13) (end 69.596 104.13) (width 0.8) (layer "B.Cu") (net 33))
 (segment (start 66.548 92.2495) (end 66.548 102.87) (width 0.8) (layer "B.Cu") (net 33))
 (segment (start 66.7275 87.62) (end 64.77 89.5775) (width 0.8) (layer "B.Cu") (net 34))
 (segment (start 64.77 89.5775) (end 64.77 104.394) (width 0.8) (layer "B.Cu") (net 34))
 (segment (start 64.77 104.394) (end 67.046 106.67) (width 0.8) (layer "B.Cu") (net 34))
 (segment (start 67.046 106.67) (end 69.596 106.67) (width 0.8) (layer "B.Cu") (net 34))
 (segment (start 68.0775 87.62) (end 66.7275 87.62) (width 0.8) (layer "B.Cu") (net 34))
 (segment (start 80.01 92.964) (end 80.01 106.924) (width 0.3) (layer "B.Cu") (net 10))
 (segment (start 84.328 93.98) (end 84.328 92.71) (width 0.3) (layer "B.Cu") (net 10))
 (segment (start 83.058 91.44) (end 81.534 91.44) (width 0.3) (layer "B.Cu") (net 10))
 (segment (start 86.36 96.52) (end 86.36 96.012) (width 0.3) (layer "B.Cu") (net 10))
 (segment (start 84.328 92.71) (end 83.058 91.44) (width 0.3) (layer "B.Cu") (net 10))
 (segment (start 81.534 91.44) (end 80.01 92.964) (width 0.3) (layer "B.Cu") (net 10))
 (segment (start 86.36 96.012) (end 84.328 93.98) (width 0.3) (layer "B.Cu") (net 10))
 (segment (start 80.01 106.924) (end 82.296 109.21) (width 0.3) (layer "B.Cu") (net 10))
 (segment (start 84.836 96.51) (end 84.836 97.536) (width 0.3) (layer "B.Cu") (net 11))
 (segment (start 84.836 97.536) (end 86.36 99.06) (width 0.3) (layer "B.Cu") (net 11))
 (segment (start 82.296 93.97) (end 84.836 96.51) (width 0.3) (layer "B.Cu") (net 11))
 (segment (start 84.846 109.22) (end 86.36 109.22) (width 0.25) (layer "B.Cu") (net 15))
 (segment (start 82.296 106.67) (end 84.846 109.22) (width 0.25) (layer "B.Cu") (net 15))
 (segment (start 84.846 106.68) (end 82.296 104.13) (width 0.25) (layer "B.Cu") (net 14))
 (segment (start 84.846 106.68) (end 86.36 106.68) (width 0.25) (layer "B.Cu") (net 14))
 (segment (start 84.328 98.542) (end 82.296 96.51) (width 0.25) (layer "B.Cu") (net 12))
 (segment (start 86.36 101.6) (end 86.36 101.551294) (width 0.25) (layer "B.Cu") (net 12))
 (segment (start 84.328 99.519294) (end 84.328 98.542) (width 0.25) (layer "B.Cu") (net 12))
 (segment (start 86.36 101.551294) (end 84.328 99.519294) (width 0.25) (layer "B.Cu") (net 12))
 (segment (start 85.344 104.14) (end 86.36 104.14) (width 0.25) (layer "B.Cu") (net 13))
 (segment (start 82.296 99.05) (end 84.582 101.336) (width 0.25) (layer "B.Cu") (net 13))
 (segment (start 84.582 103.378) (end 85.344 104.14) (width 0.25) (layer "B.Cu") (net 13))
 (segment (start 84.582 101.336) (end 84.582 103.378) (width 0.25) (layer "B.Cu") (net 13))
 (segment (start 101.092 71.12) (end 101.092 72.39) (width 0.3) (layer "B.Cu") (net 2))
 (segment (start 96.012 66.04) (end 101.092 71.12) (width 0.3) (layer "B.Cu") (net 2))
 (segment (start 85.852 64.77) (end 88.9 67.818) (width 0.3) (layer "B.Cu") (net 2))
 (segment (start 88.9 67.818) (end 88.9 68.834) (width 0.3) (layer "B.Cu") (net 2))
 (segment (start 90.678 66.04) (end 96.012 66.04) (width 0.3) (layer "B.Cu") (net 2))
 (segment (start 88.9 70.14) (end 88.9 68.834) (width 0.3) (layer "B.Cu") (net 2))
 (segment (start 85.852 64.77) (end 84.328 64.77) (width 0.3) (layer "B.Cu") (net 2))
 (segment (start 88.9 67.818) (end 90.678 66.04) (width 0.3) (layer "B.Cu") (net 2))
 (segment (start 88.646 81.28) (end 86.36 81.28) (width 0.25) (layer "B.Cu") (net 5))
 (segment (start 91.44 78.486) (end 88.646 81.28) (width 0.25) (layer "B.Cu") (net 5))
 (segment (start 91.44 70.14) (end 91.44 78.486) (width 0.25) (layer "B.Cu") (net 5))
 (segment (start 86.36 78.74) (end 85.09 78.74) (width 0.25) (layer "B.Cu") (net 1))
 (segment (start 85.09 78.74) (end 84.328 77.978) (width 0.25) (layer "B.Cu") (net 1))
 (segment (start 84.328 77.978) (end 84.328 72.39) (width 0.25) (layer "B.Cu") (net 1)))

